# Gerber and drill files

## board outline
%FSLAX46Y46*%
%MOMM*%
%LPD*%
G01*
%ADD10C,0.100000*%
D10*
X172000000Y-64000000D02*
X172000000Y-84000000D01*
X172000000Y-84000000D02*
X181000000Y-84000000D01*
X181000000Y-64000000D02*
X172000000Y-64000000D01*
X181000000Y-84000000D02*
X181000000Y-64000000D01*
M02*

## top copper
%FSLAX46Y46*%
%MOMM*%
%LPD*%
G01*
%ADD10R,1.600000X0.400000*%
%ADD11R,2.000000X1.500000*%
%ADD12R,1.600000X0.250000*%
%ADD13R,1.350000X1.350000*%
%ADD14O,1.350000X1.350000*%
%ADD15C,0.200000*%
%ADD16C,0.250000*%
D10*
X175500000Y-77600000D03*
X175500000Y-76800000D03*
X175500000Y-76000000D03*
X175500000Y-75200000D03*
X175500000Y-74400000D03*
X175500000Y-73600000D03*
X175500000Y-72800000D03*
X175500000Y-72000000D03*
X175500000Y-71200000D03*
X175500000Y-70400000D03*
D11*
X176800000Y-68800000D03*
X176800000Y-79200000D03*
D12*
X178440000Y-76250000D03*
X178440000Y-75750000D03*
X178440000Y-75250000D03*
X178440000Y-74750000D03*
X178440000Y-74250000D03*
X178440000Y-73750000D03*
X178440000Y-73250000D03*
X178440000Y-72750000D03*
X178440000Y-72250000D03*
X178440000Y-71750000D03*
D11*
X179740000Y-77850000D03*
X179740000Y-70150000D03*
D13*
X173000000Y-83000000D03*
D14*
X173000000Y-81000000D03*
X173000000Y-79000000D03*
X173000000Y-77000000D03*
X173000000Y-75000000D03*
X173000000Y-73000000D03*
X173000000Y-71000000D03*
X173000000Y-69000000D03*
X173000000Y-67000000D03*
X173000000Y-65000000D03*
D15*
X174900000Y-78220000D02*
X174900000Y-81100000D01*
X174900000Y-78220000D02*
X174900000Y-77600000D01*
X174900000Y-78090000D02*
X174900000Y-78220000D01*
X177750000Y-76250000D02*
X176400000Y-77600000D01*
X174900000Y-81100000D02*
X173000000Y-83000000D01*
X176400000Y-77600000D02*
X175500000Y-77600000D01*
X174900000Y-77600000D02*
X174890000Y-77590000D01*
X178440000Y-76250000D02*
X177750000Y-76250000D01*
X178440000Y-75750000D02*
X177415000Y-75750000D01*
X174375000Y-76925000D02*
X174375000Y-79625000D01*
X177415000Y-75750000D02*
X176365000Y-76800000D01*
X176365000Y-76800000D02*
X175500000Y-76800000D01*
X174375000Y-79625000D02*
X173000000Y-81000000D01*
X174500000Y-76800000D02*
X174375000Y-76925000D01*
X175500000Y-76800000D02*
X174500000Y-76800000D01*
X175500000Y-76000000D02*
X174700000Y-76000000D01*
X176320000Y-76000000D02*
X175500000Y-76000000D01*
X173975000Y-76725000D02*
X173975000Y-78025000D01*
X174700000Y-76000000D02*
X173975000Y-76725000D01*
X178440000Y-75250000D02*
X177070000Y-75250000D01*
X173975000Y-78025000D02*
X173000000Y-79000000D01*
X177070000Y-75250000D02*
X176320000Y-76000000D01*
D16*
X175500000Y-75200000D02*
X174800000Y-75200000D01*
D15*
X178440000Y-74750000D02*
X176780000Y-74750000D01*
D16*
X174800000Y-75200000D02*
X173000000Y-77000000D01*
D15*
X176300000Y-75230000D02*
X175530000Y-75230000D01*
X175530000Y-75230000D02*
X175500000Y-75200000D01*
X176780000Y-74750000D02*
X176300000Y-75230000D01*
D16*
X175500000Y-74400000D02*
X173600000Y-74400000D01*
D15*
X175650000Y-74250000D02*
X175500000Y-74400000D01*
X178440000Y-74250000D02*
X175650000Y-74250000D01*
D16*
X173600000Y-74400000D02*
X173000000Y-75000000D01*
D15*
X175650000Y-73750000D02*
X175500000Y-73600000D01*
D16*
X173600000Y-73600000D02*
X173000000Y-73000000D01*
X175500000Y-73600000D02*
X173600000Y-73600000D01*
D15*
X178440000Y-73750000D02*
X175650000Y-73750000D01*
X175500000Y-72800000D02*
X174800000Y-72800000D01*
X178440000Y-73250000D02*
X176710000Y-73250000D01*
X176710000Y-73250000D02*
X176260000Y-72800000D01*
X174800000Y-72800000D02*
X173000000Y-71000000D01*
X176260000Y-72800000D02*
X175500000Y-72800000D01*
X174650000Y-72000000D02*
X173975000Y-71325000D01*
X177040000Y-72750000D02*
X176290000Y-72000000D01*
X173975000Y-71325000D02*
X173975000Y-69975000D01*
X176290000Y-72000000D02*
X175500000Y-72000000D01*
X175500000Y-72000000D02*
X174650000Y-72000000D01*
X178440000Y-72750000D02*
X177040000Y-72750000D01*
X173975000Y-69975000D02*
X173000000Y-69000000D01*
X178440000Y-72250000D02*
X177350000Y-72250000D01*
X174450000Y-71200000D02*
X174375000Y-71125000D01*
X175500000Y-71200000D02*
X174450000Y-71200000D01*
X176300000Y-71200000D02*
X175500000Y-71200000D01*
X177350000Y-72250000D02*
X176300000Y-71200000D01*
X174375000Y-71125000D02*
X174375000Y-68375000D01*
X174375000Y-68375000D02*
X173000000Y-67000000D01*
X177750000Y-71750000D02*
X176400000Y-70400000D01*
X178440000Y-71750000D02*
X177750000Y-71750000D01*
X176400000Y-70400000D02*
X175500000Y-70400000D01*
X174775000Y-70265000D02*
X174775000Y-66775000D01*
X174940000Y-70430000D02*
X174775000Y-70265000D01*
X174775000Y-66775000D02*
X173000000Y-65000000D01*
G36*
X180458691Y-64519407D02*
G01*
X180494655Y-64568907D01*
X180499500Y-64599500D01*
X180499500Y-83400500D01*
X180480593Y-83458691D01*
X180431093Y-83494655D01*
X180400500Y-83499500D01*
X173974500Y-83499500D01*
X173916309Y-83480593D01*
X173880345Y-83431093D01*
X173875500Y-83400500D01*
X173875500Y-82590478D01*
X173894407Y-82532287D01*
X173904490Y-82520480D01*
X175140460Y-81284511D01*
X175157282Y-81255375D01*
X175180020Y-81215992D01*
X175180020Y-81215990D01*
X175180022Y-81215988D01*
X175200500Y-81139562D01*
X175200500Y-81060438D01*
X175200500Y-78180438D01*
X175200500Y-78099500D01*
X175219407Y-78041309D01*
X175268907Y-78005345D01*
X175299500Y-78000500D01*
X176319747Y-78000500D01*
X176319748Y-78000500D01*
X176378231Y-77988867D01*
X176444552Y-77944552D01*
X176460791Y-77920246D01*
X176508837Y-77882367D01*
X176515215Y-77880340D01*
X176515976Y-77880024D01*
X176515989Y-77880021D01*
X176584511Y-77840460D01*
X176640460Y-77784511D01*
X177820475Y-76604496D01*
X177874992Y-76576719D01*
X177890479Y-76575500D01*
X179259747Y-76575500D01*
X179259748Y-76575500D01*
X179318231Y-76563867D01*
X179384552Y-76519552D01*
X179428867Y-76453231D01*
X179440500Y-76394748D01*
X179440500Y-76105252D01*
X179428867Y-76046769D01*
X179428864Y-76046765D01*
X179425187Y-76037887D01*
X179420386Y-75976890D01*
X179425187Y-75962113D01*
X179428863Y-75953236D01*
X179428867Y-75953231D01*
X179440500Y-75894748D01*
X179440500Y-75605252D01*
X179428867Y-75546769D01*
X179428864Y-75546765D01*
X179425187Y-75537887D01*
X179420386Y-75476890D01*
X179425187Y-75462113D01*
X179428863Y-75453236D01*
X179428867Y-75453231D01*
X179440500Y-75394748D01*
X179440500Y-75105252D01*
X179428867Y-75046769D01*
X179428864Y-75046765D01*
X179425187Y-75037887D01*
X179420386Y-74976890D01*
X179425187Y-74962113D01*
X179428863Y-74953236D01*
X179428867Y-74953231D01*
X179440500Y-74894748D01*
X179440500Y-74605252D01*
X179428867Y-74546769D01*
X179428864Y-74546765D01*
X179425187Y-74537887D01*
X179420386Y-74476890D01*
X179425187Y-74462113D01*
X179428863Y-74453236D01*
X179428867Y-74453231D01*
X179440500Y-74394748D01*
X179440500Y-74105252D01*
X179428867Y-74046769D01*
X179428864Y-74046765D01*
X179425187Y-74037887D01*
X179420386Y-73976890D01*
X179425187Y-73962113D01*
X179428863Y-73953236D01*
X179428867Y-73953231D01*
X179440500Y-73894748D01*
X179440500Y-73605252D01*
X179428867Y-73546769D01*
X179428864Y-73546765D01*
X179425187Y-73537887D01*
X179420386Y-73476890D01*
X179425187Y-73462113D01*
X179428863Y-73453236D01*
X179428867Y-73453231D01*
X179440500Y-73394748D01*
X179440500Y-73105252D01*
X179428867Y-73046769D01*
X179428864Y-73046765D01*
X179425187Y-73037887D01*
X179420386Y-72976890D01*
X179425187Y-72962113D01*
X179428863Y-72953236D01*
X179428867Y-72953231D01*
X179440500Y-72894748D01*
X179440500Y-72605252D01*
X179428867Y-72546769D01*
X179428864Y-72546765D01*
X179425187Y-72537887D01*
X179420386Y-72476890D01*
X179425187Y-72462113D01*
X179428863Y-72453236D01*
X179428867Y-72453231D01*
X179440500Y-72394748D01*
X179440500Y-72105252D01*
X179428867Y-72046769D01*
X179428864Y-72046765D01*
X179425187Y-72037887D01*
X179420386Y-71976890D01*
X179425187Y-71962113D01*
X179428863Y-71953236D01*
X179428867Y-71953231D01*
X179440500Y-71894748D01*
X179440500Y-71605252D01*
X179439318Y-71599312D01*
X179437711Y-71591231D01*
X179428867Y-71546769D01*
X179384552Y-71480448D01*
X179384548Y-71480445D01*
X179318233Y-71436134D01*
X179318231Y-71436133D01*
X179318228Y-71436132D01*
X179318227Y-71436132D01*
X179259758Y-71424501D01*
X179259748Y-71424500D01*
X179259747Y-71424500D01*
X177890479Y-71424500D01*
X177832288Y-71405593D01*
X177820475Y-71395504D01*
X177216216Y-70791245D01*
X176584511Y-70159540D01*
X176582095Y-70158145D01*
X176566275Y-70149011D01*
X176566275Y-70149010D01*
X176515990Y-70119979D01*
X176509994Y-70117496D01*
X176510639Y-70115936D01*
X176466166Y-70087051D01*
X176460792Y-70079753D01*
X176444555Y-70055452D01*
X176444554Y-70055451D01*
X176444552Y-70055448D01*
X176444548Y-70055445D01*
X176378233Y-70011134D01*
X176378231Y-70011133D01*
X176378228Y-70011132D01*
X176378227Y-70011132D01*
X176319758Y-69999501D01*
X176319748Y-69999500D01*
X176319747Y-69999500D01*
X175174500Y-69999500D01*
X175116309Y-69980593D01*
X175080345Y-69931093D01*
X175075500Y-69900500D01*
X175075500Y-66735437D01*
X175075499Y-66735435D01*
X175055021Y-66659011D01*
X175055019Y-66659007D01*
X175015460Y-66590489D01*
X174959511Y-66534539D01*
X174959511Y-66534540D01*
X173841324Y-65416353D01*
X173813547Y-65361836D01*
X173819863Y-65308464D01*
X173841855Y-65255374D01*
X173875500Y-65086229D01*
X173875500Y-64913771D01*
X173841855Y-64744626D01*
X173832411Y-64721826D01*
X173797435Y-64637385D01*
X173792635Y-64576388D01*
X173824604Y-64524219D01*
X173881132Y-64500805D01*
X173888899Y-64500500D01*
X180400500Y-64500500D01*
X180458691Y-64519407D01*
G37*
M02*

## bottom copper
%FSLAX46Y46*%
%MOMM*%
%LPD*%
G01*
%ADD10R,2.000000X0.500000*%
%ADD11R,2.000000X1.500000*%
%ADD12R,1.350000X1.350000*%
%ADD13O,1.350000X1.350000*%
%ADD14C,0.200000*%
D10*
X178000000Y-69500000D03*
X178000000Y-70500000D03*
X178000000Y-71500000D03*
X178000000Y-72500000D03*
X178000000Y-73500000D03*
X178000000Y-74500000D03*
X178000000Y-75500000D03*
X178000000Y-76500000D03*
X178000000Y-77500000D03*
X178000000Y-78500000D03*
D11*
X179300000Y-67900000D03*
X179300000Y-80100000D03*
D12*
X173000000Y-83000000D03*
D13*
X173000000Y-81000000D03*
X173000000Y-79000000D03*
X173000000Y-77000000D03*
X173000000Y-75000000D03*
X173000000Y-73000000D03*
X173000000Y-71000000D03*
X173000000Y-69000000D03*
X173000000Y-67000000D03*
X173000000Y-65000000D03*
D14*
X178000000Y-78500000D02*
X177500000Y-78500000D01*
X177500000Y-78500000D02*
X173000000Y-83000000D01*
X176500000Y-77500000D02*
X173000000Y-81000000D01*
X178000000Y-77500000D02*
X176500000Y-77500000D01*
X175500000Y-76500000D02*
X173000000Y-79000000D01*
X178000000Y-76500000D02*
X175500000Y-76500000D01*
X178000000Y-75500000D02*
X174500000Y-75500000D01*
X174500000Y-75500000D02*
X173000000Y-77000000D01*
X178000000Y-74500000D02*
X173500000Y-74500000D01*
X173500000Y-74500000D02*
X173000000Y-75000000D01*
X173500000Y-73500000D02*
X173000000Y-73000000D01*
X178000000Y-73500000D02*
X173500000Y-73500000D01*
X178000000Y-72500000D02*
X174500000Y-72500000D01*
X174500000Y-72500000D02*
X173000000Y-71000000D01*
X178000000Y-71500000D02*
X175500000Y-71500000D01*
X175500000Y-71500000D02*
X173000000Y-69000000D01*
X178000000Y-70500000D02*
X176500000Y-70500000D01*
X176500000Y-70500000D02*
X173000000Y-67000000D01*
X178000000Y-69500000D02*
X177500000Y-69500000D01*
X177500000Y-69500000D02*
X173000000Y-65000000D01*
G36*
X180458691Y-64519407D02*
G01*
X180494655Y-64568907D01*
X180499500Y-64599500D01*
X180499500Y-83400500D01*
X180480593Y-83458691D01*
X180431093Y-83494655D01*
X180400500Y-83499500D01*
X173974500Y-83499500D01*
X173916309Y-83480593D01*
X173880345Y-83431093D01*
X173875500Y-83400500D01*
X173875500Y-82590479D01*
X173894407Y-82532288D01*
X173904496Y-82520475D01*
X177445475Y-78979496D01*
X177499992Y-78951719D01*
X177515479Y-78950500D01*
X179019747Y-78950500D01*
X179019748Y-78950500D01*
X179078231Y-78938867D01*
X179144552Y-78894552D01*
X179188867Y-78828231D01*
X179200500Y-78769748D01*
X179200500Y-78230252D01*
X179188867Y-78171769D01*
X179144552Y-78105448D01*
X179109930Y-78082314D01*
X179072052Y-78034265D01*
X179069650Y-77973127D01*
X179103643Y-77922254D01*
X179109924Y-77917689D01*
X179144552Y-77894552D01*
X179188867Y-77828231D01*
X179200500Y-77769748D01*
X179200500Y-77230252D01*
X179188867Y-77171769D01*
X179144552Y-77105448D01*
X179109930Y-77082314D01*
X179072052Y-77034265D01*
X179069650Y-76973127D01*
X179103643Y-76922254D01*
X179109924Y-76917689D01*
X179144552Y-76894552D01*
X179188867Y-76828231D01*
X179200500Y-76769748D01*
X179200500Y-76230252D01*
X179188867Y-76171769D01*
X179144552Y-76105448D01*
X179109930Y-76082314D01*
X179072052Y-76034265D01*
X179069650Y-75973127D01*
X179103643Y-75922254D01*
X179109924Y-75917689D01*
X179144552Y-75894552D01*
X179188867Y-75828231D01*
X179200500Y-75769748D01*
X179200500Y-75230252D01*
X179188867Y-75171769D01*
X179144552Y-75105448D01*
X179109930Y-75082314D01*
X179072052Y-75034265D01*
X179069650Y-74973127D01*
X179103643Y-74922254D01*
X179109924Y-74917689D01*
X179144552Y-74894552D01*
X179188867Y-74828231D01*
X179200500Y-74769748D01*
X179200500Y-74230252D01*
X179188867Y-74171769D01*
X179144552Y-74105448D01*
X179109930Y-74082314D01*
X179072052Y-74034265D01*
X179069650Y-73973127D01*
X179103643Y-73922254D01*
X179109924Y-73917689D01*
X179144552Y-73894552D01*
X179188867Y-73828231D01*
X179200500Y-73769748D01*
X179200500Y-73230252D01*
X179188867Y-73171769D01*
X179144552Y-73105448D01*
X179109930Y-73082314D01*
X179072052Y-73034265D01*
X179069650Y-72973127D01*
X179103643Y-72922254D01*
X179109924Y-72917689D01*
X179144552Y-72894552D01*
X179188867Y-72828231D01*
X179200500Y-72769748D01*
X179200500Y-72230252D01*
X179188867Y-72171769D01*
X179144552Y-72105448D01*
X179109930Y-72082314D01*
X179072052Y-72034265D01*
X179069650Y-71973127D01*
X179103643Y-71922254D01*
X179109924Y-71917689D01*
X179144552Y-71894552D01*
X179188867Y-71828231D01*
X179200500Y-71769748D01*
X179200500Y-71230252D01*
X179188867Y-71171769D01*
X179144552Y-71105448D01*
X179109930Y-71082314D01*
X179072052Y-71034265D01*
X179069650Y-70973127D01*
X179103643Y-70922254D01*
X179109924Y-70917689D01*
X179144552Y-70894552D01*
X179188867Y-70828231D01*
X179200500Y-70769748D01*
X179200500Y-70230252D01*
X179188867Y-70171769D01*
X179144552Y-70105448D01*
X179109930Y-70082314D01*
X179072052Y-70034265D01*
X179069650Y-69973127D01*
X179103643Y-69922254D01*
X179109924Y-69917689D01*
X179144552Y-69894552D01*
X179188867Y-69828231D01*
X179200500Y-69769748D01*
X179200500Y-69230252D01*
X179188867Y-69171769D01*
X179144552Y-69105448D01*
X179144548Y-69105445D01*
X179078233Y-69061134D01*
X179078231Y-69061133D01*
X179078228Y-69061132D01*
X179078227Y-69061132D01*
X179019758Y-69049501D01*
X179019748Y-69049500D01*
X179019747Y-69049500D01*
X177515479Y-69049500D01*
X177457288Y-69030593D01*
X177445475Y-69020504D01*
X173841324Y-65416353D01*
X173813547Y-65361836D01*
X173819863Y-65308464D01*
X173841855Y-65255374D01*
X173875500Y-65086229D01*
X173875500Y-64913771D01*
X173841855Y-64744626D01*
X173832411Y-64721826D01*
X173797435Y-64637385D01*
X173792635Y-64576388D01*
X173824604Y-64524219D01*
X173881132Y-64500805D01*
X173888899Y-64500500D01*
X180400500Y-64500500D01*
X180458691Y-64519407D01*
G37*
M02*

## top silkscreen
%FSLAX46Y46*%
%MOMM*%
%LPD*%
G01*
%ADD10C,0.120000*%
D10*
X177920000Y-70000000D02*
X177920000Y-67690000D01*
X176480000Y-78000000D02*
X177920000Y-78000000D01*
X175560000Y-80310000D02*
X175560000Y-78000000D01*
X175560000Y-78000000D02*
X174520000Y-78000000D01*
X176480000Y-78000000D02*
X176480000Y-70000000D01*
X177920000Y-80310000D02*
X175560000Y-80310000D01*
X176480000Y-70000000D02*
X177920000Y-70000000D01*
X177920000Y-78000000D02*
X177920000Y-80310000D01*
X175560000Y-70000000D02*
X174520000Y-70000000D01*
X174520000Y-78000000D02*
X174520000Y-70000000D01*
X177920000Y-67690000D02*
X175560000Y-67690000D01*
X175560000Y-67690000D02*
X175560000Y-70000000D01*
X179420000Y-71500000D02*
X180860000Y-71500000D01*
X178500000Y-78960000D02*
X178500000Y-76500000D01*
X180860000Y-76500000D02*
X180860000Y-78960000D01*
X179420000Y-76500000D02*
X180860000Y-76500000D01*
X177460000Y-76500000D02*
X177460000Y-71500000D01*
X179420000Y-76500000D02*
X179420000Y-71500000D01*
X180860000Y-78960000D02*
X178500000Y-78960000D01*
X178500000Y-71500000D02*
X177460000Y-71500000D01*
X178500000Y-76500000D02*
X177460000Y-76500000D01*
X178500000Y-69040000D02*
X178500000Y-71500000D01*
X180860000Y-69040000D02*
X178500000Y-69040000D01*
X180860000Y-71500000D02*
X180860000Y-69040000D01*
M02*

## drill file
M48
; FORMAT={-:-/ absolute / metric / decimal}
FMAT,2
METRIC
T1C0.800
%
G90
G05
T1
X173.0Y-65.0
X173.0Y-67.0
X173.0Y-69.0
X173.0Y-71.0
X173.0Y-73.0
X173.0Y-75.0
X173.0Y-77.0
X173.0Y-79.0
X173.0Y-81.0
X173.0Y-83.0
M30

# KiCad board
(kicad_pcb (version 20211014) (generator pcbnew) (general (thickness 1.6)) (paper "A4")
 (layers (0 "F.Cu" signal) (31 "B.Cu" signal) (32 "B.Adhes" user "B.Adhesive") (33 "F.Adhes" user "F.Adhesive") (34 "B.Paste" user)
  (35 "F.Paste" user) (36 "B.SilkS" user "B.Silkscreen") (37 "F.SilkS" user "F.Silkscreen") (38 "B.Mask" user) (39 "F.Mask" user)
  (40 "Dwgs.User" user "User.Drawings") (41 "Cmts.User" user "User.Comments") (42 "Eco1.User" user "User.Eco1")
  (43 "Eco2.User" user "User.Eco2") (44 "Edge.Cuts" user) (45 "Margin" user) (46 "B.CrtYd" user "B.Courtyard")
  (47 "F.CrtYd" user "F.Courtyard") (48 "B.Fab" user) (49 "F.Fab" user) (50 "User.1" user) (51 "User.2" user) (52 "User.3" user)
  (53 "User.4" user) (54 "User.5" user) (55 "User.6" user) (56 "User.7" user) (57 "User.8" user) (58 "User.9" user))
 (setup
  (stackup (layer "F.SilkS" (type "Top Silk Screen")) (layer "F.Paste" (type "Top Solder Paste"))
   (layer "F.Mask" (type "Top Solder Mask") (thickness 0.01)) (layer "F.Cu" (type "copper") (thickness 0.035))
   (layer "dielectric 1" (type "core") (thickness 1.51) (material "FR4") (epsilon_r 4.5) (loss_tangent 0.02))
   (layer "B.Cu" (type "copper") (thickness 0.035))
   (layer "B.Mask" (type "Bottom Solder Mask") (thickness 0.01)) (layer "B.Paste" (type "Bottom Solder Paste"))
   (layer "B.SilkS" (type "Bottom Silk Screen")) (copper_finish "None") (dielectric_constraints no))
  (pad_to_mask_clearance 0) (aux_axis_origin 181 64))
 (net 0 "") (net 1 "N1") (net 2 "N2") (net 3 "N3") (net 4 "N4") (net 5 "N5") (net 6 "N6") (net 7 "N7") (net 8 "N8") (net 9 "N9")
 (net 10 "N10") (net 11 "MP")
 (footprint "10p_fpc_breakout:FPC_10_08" (layer "F.Cu") (at 175.5 74 90)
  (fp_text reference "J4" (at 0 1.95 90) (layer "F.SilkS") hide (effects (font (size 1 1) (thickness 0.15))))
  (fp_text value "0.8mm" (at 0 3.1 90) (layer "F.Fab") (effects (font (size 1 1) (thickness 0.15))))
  (fp_line (start 4 2.42) (end 6.31 2.42) (layer "F.SilkS") (width 0.12))
  (fp_line (start -4 0.98) (end -4 2.42) (layer "F.SilkS") (width 0.12))
  (fp_line (start -6.31 0.06) (end -4 0.06) (layer "F.SilkS") (width 0.12))
  (fp_line (start -4 0.06) (end -4 -0.98) (layer "F.SilkS") (width 0.12))
  (fp_line (start -4 0.98) (end 4 0.98) (layer "F.SilkS") (width 0.12))
  (fp_line (start -6.31 2.42) (end -6.31 0.06) (layer "F.SilkS") (width 0.12))
  (fp_line (start 4 0.98) (end 4 2.42) (layer "F.SilkS") (width 0.12))
  (fp_line (start -4 2.42) (end -6.31 2.42) (layer "F.SilkS") (width 0.12))
  (fp_line (start 4 0.06) (end 4 -0.98) (layer "F.SilkS") (width 0.12))
  (fp_line (start -4 -0.98) (end 4 -0.98) (layer "F.SilkS") (width 0.12))
  (fp_line (start 6.31 2.42) (end 6.31 0.06) (layer "F.SilkS") (width 0.12))
  (fp_line (start 6.31 0.06) (end 4 0.06) (layer "F.SilkS") (width 0.12))
  (pad "1" smd rect (at -3.6 0 90) (size 0.4 1.6) (layers "F.Cu" "F.Paste" "F.Mask") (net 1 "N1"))
  (pad "2" smd rect (at -2.8 0 90) (size 0.4 1.6) (layers "F.Cu" "F.Paste" "F.Mask") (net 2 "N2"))
  (pad "3" smd rect (at -2 0 90) (size 0.4 1.6) (layers "F.Cu" "F.Paste" "F.Mask") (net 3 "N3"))
  (pad "4" smd rect (at -1.2 0 90) (size 0.4 1.6) (layers "F.Cu" "F.Paste" "F.Mask") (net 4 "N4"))
  (pad "5" smd rect (at -0.4 0 90) (size 0.4 1.6) (layers "F.Cu" "F.Paste" "F.Mask") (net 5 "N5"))
  (pad "6" smd rect (at 0.4 0 90) (size 0.4 1.6) (layers "F.Cu" "F.Paste" "F.Mask") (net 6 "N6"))
  (pad "7" smd rect (at 1.2 0 90) (size 0.4 1.6) (layers "F.Cu" "F.Paste" "F.Mask") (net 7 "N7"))
  (pad "8" smd rect (at 2 0 90) (size 0.4 1.6) (layers "F.Cu" "F.Paste" "F.Mask") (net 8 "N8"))
  (pad "9" smd rect (at 2.8 0 90) (size 0.4 1.6) (layers "F.Cu" "F.Paste" "F.Mask") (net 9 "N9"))
  (pad "10" smd rect (at 3.6 0 90) (size 0.4 1.6) (layers "F.Cu" "F.Paste" "F.Mask") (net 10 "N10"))
  (pad "MP" smd rect (at 5.2 1.3 90) (size 1.5 2) (layers "F.Cu" "F.Paste" "F.Mask") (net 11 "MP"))
  (pad "MP" smd rect (at -5.2 1.3 90) (size 1.5 2) (layers "F.Cu" "F.Paste" "F.Mask") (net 11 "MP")))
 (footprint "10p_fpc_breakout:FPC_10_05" (layer "F.Cu") (at 178.44 74 90)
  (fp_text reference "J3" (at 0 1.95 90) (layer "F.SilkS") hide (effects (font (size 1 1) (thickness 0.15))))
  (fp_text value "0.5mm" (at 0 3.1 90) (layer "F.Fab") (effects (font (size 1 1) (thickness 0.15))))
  (fp_line (start 2.5 0.98) (end 2.5 2.42) (layer "F.SilkS") (width 0.12))
  (fp_line (start -4.96 0.06) (end -2.5 0.06) (layer "F.SilkS") (width 0.12))
  (fp_line (start -2.5 2.42) (end -4.96 2.42) (layer "F.SilkS") (width 0.12))
  (fp_line (start -2.5 0.98) (end -2.5 2.42) (layer "F.SilkS") (width 0.12))
  (fp_line (start -2.5 -0.98) (end 2.5 -0.98) (layer "F.SilkS") (width 0.12))
  (fp_line (start -2.5 0.98) (end 2.5 0.98) (layer "F.SilkS") (width 0.12))
  (fp_line (start -4.96 2.42) (end -4.96 0.06) (layer "F.SilkS") (width 0.12))
  (fp_line (start 2.5 0.06) (end 2.5 -0.98) (layer "F.SilkS") (width 0.12))
  (fp_line (start -2.5 0.06) (end -2.5 -0.98) (layer "F.SilkS") (width 0.12))
  (fp_line (start 4.96 0.06) (end 2.5 0.06) (layer "F.SilkS") (width 0.12))
  (fp_line (start 4.96 2.42) (end 4.96 0.06) (layer "F.SilkS") (width 0.12))
  (fp_line (start 2.5 2.42) (end 4.96 2.42) (layer "F.SilkS") (width 0.12))
  (pad "1" smd rect (at -2.25 0 90) (size 0.25 1.6) (layers "F.Cu" "F.Paste" "F.Mask") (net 1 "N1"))
  (pad "2" smd rect (at -1.75 0 90) (size 0.25 1.6) (layers "F.Cu" "F.Paste" "F.Mask") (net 2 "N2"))
  (pad "3" smd rect (at -1.25 0 90) (size 0.25 1.6) (layers "F.Cu" "F.Paste" "F.Mask") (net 3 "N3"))
  (pad "4" smd rect (at -0.75 0 90) (size 0.25 1.6) (layers "F.Cu" "F.Paste" "F.Mask") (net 4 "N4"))
  (pad "5" smd rect (at -0.25 0 90) (size 0.25 1.6) (layers "F.Cu" "F.Paste" "F.Mask") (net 5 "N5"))
  (pad "6" smd rect (at 0.25 0 90) (size 0.25 1.6) (layers "F.Cu" "F.Paste" "F.Mask") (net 6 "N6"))
  (pad "7" smd rect (at 0.75 0 90) (size 0.25 1.6) (layers "F.Cu" "F.Paste" "F.Mask") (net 7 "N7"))
  (pad "8" smd rect (at 1.25 0 90) (size 0.25 1.6) (layers "F.Cu" "F.Paste" "F.Mask") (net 8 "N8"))
  (pad "9" smd rect (at 1.75 0 90) (size 0.25 1.6) (layers "F.Cu" "F.Paste" "F.Mask") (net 9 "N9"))
  (pad "10" smd rect (at 2.25 0 90) (size 0.25 1.6) (layers "F.Cu" "F.Paste" "F.Mask") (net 10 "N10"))
  (pad "MP" smd rect (at -3.85 1.3 90) (size 1.5 2) (layers "F.Cu" "F.Paste" "F.Mask") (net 11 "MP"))
  (pad "MP" smd rect (at 3.85 1.3 90) (size 1.5 2) (layers "F.Cu" "F.Paste" "F.Mask") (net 11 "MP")))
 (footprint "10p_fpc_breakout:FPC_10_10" (layer "B.Cu") (at 178 74 -90)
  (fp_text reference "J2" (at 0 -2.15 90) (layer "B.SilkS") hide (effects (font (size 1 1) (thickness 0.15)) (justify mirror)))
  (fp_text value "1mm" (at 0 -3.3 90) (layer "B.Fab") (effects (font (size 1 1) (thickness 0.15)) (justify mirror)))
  (pad "1" smd rect (at -4.5 0 270) (size 0.5 2) (layers "B.Cu" "B.Paste" "B.Mask") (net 10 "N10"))
  (pad "2" smd rect (at -3.5 0 270) (size 0.5 2) (layers "B.Cu" "B.Paste" "B.Mask") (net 9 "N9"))
  (pad "3" smd rect (at -2.5 0 270) (size 0.5 2) (layers "B.Cu" "B.Paste" "B.Mask") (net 8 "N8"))
  (pad "4" smd rect (at -1.5 0 270) (size 0.5 2) (layers "B.Cu" "B.Paste" "B.Mask") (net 7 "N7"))
  (pad "5" smd rect (at -0.5 0 270) (size 0.5 2) (layers "B.Cu" "B.Paste" "B.Mask") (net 6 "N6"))
  (pad "6" smd rect (at 0.5 0 270) (size 0.5 2) (layers "B.Cu" "B.Paste" "B.Mask") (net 5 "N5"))
  (pad "7" smd rect (at 1.5 0 270) (size 0.5 2) (layers "B.Cu" "B.Paste" "B.Mask") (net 4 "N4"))
  (pad "8" smd rect (at 2.5 0 270) (size 0.5 2) (layers "B.Cu" "B.Paste" "B.Mask") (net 3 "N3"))
  (pad "9" smd rect (at 3.5 0 270) (size 0.5 2) (layers "B.Cu" "B.Paste" "B.Mask") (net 2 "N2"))
  (pad "10" smd rect (at 4.5 0 270) (size 0.5 2) (layers "B.Cu" "B.Paste" "B.Mask") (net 1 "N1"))
  (pad "MP" smd rect (at -6.1 -1.3 270) (size 1.5 2) (layers "B.Cu" "B.Paste" "B.Mask") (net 11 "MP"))
  (pad "MP" smd rect (at 6.1 -1.3 270) (size 1.5 2) (layers "B.Cu" "B.Paste" "B.Mask") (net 11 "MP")))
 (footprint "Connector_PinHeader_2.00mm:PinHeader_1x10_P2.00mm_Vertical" (layer "B.Cu") (at 173 83)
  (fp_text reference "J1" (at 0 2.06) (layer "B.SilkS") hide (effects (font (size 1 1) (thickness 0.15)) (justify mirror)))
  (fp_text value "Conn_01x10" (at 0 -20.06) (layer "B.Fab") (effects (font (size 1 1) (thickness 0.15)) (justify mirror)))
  (pad "1" thru_hole rect (at 0 0) (size 1.35 1.35) (drill 0.8) (layers *.Cu *.Mask) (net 1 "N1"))
  (pad "2" thru_hole oval (at 0 -2) (size 1.35 1.35) (drill 0.8) (layers *.Cu *.Mask) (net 2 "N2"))
  (pad "3" thru_hole oval (at 0 -4) (size 1.35 1.35) (drill 0.8) (layers *.Cu *.Mask) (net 3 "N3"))
  (pad "4" thru_hole oval (at 0 -6) (size 1.35 1.35) (drill 0.8) (layers *.Cu *.Mask) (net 4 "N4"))
  (pad "5" thru_hole oval (at 0 -8) (size 1.35 1.35) (drill 0.8) (layers *.Cu *.Mask) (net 5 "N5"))
  (pad "6" thru_hole oval (at 0 -10) (size 1.35 1.35) (drill 0.8) (layers *.Cu *.Mask) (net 6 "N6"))
  (pad "7" thru_hole oval (at 0 -12) (size 1.35 1.35) (drill 0.8) (layers *.Cu *.Mask) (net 7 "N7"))
  (pad "8" thru_hole oval (at 0 -14) (size 1.35 1.35) (drill 0.8) (layers *.Cu *.Mask) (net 8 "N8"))
  (pad "9" thru_hole oval (at 0 -16) (size 1.35 1.35) (drill 0.8) (layers *.Cu *.Mask) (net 9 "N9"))
  (pad "10" thru_hole oval (at 0 -18) (size 1.35 1.35) (drill 0.8) (layers *.Cu *.Mask) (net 10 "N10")))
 (gr_line (start 172 64) (end 172 84) (layer "Edge.Cuts") (width 0.1))
 (gr_line (start 172 84) (end 181 84) (layer "Edge.Cuts") (width 0.1))
 (gr_line (start 181 64) (end 172 64) (layer "Edge.Cuts") (width 0.1))
 (gr_line (start 181 84) (end 181 64) (layer "Edge.Cuts") (width 0.1))
 (segment (start 174.9 78.22) (end 174.9 81.1) (width 0.2) (layer "F.Cu") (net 1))
 (segment (start 174.9 78.22) (end 174.9 77.6) (width 0.2) (layer "F.Cu") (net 1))
 (segment (start 174.9 78.09) (end 174.9 78.22) (width 0.2) (layer "F.Cu") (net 1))
 (segment (start 177.75 76.25) (end 176.4 77.6) (width 0.2) (layer "F.Cu") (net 1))
 (segment (start 174.9 81.1) (end 173 83) (width 0.2) (layer "F.Cu") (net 1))
 (segment (start 176.4 77.6) (end 175.5 77.6) (width 0.2) (layer "F.Cu") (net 1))
 (segment (start 174.9 77.6) (end 174.89 77.59) (width 0.2) (layer "F.Cu") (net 1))
 (segment (start 178.44 76.25) (end 177.75 76.25) (width 0.2) (layer "F.Cu") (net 1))
 (segment (start 178 78.5) (end 177.5 78.5) (width 0.2) (layer "B.Cu") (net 1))
 (segment (start 177.5 78.5) (end 173 83) (width 0.2) (layer "B.Cu") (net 1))
 (segment (start 178.44 75.75) (end 177.415 75.75) (width 0.2) (layer "F.Cu") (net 2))
 (segment (start 174.375 76.925) (end 174.375 79.625) (width 0.2) (layer "F.Cu") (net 2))
 (segment (start 177.415 75.75) (end 176.365 76.8) (width 0.2) (layer "F.Cu") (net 2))
 (segment (start 176.365 76.8) (end 175.5 76.8) (width 0.2) (layer "F.Cu") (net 2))
 (segment (start 174.375 79.625) (end 173 81) (width 0.2) (layer "F.Cu") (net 2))
 (segment (start 174.5 76.8) (end 174.375 76.925) (width 0.2) (layer "F.Cu") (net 2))
 (segment (start 175.5 76.8) (end 174.5 76.8) (width 0.2) (layer "F.Cu") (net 2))
 (segment (start 176.5 77.5) (end 173 81) (width 0.2) (layer "B.Cu") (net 2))
 (segment (start 178 77.5) (end 176.5 77.5) (width 0.2) (layer "B.Cu") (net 2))
 (segment (start 175.5 76) (end 174.7 76) (width 0.2) (layer "F.Cu") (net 3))
 (segment (start 176.32 76) (end 175.5 76) (width 0.2) (layer "F.Cu") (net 3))
 (segment (start 173.975 76.725) (end 173.975 78.025) (width 0.2) (layer "F.Cu") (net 3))
 (segment (start 174.7 76) (end 173.975 76.725) (width 0.2) (layer "F.Cu") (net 3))
 (segment (start 178.44 75.25) (end 177.07 75.25) (width 0.2) (layer "F.Cu") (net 3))
 (segment (start 173.975 78.025) (end 173 79) (width 0.2) (layer "F.Cu") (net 3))
 (segment (start 177.07 75.25) (end 176.32 76) (width 0.2) (layer "F.Cu") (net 3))
 (segment (start 175.5 76.5) (end 173 79) (width 0.2) (layer "B.Cu") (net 3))
 (segment (start 178 76.5) (end 175.5 76.5) (width 0.2) (layer "B.Cu") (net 3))
 (segment (start 175.5 75.2) (end 174.8 75.2) (width 0.25) (layer "F.Cu") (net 4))
 (segment (start 178.44 74.75) (end 176.78 74.75) (width 0.2) (layer "F.Cu") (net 4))
 (segment (start 174.8 75.2) (end 173 77) (width 0.25) (layer "F.Cu") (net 4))
 (segment (start 176.3 75.23) (end 175.53 75.23) (width 0.2) (layer "F.Cu") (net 4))
 (segment (start 175.53 75.23) (end 175.5 75.2) (width 0.2) (layer "F.Cu") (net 4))
 (segment (start 176.78 74.75) (end 176.3 75.23) (width 0.2) (layer "F.Cu") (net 4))
 (segment (start 178 75.5) (end 174.5 75.5) (width 0.2) (layer "B.Cu") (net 4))
 (segment (start 174.5 75.5) (end 173 77) (width 0.2) (layer "B.Cu") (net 4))
 (segment (start 175.5 74.4) (end 173.6 74.4) (width 0.25) (layer "F.Cu") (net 5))
 (segment (start 175.65 74.25) (end 175.5 74.4) (width 0.2) (layer "F.Cu") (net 5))
 (segment (start 178.44 74.25) (end 175.65 74.25) (width 0.2) (layer "F.Cu") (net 5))
 (segment (start 173.6 74.4) (end 173 75) (width 0.25) (layer "F.Cu") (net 5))
 (segment (start 178 74.5) (end 173.5 74.5) (width 0.2) (layer "B.Cu") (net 5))
 (segment (start 173.5 74.5) (end 173 75) (width 0.2) (layer "B.Cu") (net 5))
 (segment (start 175.65 73.75) (end 175.5 73.6) (width 0.2) (layer "F.Cu") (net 6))
 (segment (start 173.6 73.6) (end 173 73) (width 0.25) (layer "F.Cu") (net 6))
 (segment (start 175.5 73.6) (end 173.6 73.6) (width 0.25) (layer "F.Cu") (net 6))
 (segment (start 178.44 73.75) (end 175.65 73.75) (width 0.2) (layer "F.Cu") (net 6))
 (segment (start 173.5 73.5) (end 173 73) (width 0.2) (layer "B.Cu") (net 6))
 (segment (start 178 73.5) (end 173.5 73.5) (width 0.2) (layer "B.Cu") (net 6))
 (segment (start 175.5 72.8) (end 174.8 72.8) (width 0.2) (layer "F.Cu") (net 7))
 (segment (start 178.44 73.25) (end 176.71 73.25) (width 0.2) (layer "F.Cu") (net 7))
 (segment (start 176.71 73.25) (end 176.26 72.8) (width 0.2) (layer "F.Cu") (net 7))
 (segment (start 174.8 72.8) (end 173 71) (width 0.2) (layer "F.Cu") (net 7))
 (segment (start 176.26 72.8) (end 175.5 72.8) (width 0.2) (layer "F.Cu") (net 7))
 (segment (start 178 72.5) (end 174.5 72.5) (width 0.2) (layer "B.Cu") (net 7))
 (segment (start 174.5 72.5) (end 173 71) (width 0.2) (layer "B.Cu") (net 7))
 (segment (start 174.65 72) (end 173.975 71.325) (width 0.2) (layer "F.Cu") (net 8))
 (segment (start 177.04 72.75) (end 176.29 72) (width 0.2) (layer "F.Cu") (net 8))
 (segment (start 173.975 71.325) (end 173.975 69.975) (width 0.2) (layer "F.Cu") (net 8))
 (segment (start 176.29 72) (end 175.5 72) (width 0.2) (layer "F.Cu") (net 8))
 (segment (start 175.5 72) (end 174.65 72) (width 0.2) (layer "F.Cu") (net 8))
 (segment (start 178.44 72.75) (end 177.04 72.75) (width 0.2) (layer "F.Cu") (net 8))
 (segment (start 173.975 69.975) (end 173 69) (width 0.2) (layer "F.Cu") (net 8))
 (segment (start 178 71.5) (end 175.5 71.5) (width 0.2) (layer "B.Cu") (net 8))
 (segment (start 175.5 71.5) (end 173 69) (width 0.2) (layer "B.Cu") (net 8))
 (segment (start 178.44 72.25) (end 177.35 72.25) (width 0.2) (layer "F.Cu") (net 9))
 (segment (start 174.45 71.2) (end 174.375 71.125) (width 0.2) (layer "F.Cu") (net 9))
 (segment (start 175.5 71.2) (end 174.45 71.2) (width 0.2) (layer "F.Cu") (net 9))
 (segment (start 176.3 71.2) (end 175.5 71.2) (width 0.2) (layer "F.Cu") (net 9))
 (segment (start 177.35 72.25) (end 176.3 71.2) (width 0.2) (layer "F.Cu") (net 9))
 (segment (start 174.375 71.125) (end 174.375 68.375) (width 0.2) (layer "F.Cu") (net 9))
 (segment (start 174.375 68.375) (end 173 67) (width 0.2) (layer "F.Cu") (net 9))
 (segment (start 178 70.5) (end 176.5 70.5) (width 0.2) (layer "B.Cu") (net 9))
 (segment (start 176.5 70.5) (end 173 67) (width 0.2) (layer "B.Cu") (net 9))
 (segment (start 177.75 71.75) (end 176.4 70.4) (width 0.2) (layer "F.Cu") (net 10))
 (segment (start 178.44 71.75) (end 177.75 71.75) (width 0.2) (layer "F.Cu") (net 10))
 (segment (start 176.4 70.4) (end 175.5 70.4) (width 0.2) (layer "F.Cu") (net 10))
 (segment (start 174.775 70.265) (end 174.775 66.775) (width 0.2) (layer "F.Cu") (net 10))
 (segment (start 174.94 70.43) (end 174.775 70.265) (width 0.2) (layer "F.Cu") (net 10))
 (segment (start 174.775 66.775) (end 173 65) (width 0.2) (layer "F.Cu") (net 10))
 (segment (start 178 69.5) (end 177.5 69.5) (width 0.2) (layer "B.Cu") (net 10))
 (segment (start 177.5 69.5) (end 173 65) (width 0.2) (layer "B.Cu") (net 10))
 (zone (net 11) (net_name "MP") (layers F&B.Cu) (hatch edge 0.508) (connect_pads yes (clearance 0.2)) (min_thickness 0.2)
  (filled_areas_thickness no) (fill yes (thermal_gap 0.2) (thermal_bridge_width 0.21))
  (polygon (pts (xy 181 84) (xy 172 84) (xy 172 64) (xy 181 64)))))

